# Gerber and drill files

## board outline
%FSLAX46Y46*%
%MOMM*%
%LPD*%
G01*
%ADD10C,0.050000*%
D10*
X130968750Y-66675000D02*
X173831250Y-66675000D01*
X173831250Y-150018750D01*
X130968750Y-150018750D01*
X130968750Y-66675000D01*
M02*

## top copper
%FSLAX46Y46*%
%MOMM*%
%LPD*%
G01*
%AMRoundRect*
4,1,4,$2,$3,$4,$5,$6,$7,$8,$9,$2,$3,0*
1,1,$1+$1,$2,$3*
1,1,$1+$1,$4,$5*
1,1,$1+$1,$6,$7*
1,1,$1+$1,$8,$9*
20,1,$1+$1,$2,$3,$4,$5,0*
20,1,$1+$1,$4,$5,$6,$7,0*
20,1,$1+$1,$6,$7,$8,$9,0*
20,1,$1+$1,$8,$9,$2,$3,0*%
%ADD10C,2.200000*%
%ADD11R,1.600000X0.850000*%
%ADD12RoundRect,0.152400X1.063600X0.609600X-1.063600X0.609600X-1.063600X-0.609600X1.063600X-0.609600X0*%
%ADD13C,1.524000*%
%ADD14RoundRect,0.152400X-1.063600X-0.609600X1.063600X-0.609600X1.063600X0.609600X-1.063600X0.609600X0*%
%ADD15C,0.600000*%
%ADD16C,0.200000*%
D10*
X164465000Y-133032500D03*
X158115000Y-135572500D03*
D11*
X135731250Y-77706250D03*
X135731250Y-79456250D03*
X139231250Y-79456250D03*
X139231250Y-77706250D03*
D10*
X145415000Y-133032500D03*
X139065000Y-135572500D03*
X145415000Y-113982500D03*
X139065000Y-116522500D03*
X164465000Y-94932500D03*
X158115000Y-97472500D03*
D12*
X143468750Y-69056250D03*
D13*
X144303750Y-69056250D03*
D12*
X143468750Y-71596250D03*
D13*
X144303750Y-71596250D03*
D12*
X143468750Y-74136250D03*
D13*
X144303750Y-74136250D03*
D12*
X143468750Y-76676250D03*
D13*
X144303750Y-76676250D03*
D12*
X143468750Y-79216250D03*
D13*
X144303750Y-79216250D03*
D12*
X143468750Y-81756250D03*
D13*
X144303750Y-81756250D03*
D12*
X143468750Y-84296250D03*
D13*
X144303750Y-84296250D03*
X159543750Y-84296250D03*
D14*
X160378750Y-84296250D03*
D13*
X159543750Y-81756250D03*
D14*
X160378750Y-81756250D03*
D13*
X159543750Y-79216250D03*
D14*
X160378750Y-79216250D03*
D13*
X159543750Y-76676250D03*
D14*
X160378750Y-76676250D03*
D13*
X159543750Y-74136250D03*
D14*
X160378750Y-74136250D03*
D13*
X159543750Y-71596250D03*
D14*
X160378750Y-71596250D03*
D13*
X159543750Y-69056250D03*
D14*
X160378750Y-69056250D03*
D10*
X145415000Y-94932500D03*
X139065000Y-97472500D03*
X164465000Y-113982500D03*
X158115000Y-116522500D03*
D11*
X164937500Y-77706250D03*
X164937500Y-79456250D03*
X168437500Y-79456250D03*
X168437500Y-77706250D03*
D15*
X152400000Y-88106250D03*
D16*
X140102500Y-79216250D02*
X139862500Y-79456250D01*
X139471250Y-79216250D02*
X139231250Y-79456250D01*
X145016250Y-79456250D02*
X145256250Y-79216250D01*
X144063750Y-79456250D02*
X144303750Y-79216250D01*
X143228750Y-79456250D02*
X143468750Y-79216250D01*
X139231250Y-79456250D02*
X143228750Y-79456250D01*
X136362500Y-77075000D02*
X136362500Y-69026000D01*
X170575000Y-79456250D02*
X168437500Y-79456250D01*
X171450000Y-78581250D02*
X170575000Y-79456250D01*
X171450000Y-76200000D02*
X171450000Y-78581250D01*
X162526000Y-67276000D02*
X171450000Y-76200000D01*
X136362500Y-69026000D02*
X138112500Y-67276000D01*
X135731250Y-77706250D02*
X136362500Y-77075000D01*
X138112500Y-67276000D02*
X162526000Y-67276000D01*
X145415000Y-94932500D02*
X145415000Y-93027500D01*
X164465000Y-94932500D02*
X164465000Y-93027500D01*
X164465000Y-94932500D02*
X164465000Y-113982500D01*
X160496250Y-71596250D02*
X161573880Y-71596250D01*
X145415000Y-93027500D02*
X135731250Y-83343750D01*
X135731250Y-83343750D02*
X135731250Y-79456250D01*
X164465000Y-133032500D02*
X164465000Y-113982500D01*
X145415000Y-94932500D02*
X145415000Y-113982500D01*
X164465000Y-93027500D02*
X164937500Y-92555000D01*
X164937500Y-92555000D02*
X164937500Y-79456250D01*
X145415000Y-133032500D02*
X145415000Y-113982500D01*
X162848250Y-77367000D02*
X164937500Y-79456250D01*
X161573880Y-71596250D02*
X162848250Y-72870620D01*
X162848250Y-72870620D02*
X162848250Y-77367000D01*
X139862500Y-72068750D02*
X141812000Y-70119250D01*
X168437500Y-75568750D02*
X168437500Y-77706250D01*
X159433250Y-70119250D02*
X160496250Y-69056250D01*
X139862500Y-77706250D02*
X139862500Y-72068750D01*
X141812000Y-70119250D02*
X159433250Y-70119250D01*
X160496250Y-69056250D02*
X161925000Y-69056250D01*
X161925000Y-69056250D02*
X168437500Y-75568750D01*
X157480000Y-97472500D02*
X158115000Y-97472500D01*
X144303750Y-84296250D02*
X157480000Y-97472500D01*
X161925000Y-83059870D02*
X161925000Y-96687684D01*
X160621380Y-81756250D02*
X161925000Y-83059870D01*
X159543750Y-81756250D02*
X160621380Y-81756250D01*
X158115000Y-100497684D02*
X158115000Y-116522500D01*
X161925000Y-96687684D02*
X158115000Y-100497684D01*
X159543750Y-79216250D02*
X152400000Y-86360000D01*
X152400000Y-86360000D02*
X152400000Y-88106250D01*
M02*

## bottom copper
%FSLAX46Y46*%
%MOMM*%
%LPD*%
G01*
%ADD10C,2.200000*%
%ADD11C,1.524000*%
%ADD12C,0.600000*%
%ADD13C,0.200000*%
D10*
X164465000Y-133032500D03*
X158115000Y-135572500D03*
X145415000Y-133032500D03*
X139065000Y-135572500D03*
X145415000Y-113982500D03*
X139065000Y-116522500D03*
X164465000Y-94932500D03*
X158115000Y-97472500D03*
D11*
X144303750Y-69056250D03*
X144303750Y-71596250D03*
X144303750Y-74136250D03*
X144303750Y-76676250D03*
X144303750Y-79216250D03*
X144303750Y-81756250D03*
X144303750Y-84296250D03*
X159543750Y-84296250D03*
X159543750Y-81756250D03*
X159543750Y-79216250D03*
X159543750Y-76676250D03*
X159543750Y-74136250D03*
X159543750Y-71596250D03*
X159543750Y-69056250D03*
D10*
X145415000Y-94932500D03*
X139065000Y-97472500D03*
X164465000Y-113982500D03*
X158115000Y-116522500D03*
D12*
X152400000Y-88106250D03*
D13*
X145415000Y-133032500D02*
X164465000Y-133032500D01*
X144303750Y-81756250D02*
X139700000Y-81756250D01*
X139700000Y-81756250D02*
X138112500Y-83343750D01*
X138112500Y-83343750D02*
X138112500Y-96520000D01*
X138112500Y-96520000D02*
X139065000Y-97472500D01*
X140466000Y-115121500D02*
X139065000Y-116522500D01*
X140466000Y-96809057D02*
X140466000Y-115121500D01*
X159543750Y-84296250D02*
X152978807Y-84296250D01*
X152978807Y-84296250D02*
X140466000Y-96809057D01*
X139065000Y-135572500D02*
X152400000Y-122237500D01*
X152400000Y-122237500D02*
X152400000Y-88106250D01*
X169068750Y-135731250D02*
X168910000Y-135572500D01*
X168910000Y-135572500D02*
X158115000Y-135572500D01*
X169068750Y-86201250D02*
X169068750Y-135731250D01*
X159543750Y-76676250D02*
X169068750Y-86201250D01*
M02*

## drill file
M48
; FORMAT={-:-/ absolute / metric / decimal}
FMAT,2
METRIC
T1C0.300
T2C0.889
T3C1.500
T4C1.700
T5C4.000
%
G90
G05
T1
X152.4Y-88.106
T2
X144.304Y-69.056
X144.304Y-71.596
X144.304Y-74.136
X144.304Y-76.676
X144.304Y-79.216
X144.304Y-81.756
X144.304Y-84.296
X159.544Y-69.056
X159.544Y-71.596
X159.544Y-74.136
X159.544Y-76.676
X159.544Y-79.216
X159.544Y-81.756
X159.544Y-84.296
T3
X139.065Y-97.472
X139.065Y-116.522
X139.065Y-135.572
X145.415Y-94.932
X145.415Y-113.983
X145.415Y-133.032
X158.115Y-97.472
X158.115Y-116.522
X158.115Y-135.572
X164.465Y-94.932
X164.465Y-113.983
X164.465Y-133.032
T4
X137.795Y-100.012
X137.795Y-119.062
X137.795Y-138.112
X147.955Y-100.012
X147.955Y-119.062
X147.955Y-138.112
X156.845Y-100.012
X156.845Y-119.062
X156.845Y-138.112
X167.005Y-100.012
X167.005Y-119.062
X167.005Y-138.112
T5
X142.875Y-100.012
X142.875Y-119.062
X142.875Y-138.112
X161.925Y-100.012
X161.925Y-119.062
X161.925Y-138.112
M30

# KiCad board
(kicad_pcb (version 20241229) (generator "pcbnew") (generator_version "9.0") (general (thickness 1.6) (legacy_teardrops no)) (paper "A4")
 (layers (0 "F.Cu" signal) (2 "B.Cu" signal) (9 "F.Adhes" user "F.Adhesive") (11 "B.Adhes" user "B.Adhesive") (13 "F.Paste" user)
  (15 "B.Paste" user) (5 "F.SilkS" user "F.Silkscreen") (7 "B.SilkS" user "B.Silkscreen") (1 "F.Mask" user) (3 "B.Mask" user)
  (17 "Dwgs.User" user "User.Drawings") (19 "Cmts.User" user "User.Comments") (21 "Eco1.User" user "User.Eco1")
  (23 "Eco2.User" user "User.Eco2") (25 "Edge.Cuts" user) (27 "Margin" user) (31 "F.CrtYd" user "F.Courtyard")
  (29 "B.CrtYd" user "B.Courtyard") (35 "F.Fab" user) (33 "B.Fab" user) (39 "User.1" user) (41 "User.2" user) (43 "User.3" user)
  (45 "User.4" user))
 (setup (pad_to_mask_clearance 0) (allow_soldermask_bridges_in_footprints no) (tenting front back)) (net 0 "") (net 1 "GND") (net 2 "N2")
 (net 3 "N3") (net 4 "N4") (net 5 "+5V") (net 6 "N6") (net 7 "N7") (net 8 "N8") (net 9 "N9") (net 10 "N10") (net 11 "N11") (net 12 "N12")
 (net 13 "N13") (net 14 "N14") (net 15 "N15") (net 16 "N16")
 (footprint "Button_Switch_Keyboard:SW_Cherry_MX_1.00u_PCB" (layer "F.Cu") (at 164.465 133.0325)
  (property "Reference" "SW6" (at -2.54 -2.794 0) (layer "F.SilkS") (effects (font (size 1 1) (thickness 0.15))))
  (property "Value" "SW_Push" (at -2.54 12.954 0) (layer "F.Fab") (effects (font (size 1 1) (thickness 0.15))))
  (pad "" np_thru_hole circle (at -7.62 5.08) (size 1.7 1.7) (drill 1.7) (layers "*.Cu" "*.Mask"))
  (pad "" np_thru_hole circle (at -2.54 5.08) (size 4 4) (drill 4) (layers "*.Cu" "*.Mask"))
  (pad "" np_thru_hole circle (at 2.54 5.08) (size 1.7 1.7) (drill 1.7) (layers "*.Cu" "*.Mask"))
  (pad "1" thru_hole circle (at 0 0) (size 2.2 2.2) (drill 1.5) (layers "*.Cu" "*.Mask") (remove_unused_layers no) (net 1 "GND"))
  (pad "2" thru_hole circle (at -6.35 2.54) (size 2.2 2.2) (drill 1.5) (layers "*.Cu" "*.Mask") (remove_unused_layers no) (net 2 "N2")))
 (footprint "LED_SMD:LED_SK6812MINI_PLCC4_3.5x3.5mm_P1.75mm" (layer "F.Cu") (at 137.48125 78.58125)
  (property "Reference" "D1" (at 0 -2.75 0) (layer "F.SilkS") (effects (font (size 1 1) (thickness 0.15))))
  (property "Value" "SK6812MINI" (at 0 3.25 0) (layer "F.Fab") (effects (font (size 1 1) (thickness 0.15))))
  (pad "1" smd rect (at -1.75 -0.875) (size 1.6 0.85) (layers "F.Cu" "F.Mask" "F.Paste") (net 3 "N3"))
  (pad "2" smd rect (at -1.75 0.875) (size 1.6 0.85) (layers "F.Cu" "F.Mask" "F.Paste") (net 1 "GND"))
  (pad "3" smd rect (at 1.75 0.875) (size 1.6 0.85) (layers "F.Cu" "F.Mask" "F.Paste") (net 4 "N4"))
  (pad "4" smd rect (at 1.75 -0.875) (size 1.6 0.85) (layers "F.Cu" "F.Mask" "F.Paste") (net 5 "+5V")))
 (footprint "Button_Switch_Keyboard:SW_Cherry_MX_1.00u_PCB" (layer "F.Cu") (at 145.415 133.0325)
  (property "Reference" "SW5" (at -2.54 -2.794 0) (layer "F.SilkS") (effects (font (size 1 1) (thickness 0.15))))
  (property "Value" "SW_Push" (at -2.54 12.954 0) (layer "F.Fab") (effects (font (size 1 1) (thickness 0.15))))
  (pad "" np_thru_hole circle (at -7.62 5.08) (size 1.7 1.7) (drill 1.7) (layers "*.Cu" "*.Mask"))
  (pad "" np_thru_hole circle (at -2.54 5.08) (size 4 4) (drill 4) (layers "*.Cu" "*.Mask"))
  (pad "" np_thru_hole circle (at 2.54 5.08) (size 1.7 1.7) (drill 1.7) (layers "*.Cu" "*.Mask"))
  (pad "1" thru_hole circle (at 0 0) (size 2.2 2.2) (drill 1.5) (layers "*.Cu" "*.Mask") (remove_unused_layers no) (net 1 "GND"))
  (pad "2" thru_hole circle (at -6.35 2.54) (size 2.2 2.2) (drill 1.5) (layers "*.Cu" "*.Mask") (remove_unused_layers no) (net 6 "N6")))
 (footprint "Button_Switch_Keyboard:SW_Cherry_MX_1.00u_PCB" (layer "F.Cu") (at 145.415 113.9825)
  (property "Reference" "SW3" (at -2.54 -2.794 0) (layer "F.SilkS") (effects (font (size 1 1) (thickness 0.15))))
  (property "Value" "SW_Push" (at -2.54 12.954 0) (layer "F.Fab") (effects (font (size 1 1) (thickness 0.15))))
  (pad "" np_thru_hole circle (at -7.62 5.08) (size 1.7 1.7) (drill 1.7) (layers "*.Cu" "*.Mask"))
  (pad "" np_thru_hole circle (at -2.54 5.08) (size 4 4) (drill 4) (layers "*.Cu" "*.Mask"))
  (pad "" np_thru_hole circle (at 2.54 5.08) (size 1.7 1.7) (drill 1.7) (layers "*.Cu" "*.Mask"))
  (pad "1" thru_hole circle (at 0 0) (size 2.2 2.2) (drill 1.5) (layers "*.Cu" "*.Mask") (remove_unused_layers no) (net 1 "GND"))
  (pad "2" thru_hole circle (at -6.35 2.54) (size 2.2 2.2) (drill 1.5) (layers "*.Cu" "*.Mask") (remove_unused_layers no) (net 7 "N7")))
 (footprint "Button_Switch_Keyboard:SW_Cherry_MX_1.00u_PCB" (layer "F.Cu") (at 164.465 94.9325)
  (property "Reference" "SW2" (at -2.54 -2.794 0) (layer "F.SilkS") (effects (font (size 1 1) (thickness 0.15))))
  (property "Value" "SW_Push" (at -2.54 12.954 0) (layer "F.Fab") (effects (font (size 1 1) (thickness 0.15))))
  (pad "" np_thru_hole circle (at -7.62 5.08) (size 1.7 1.7) (drill 1.7) (layers "*.Cu" "*.Mask"))
  (pad "" np_thru_hole circle (at -2.54 5.08) (size 4 4) (drill 4) (layers "*.Cu" "*.Mask"))
  (pad "" np_thru_hole circle (at 2.54 5.08) (size 1.7 1.7) (drill 1.7) (layers "*.Cu" "*.Mask"))
  (pad "1" thru_hole circle (at 0 0) (size 2.2 2.2) (drill 1.5) (layers "*.Cu" "*.Mask") (remove_unused_layers no) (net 1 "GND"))
  (pad "2" thru_hole circle (at -6.35 2.54) (size 2.2 2.2) (drill 1.5) (layers "*.Cu" "*.Mask") (remove_unused_layers no) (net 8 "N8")))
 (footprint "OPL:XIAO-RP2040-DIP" (layer "F.Cu") (at 151.92375 76.67625)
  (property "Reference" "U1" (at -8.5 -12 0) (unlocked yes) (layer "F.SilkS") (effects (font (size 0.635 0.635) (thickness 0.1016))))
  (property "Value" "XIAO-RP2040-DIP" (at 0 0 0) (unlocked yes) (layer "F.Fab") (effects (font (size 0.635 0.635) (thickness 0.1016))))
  (pad "1" smd roundrect (at -8.455 -7.62 180) (size 2.432 1.524) (layers "F.Cu" "F.Mask") (roundrect_rratio 0.1) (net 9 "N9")
   (thermal_bridge_angle 45))
  (pad "1" thru_hole circle (at -7.62 -7.62 180) (size 1.524 1.524) (drill 0.889) (layers "*.Cu" "*.Mask") (remove_unused_layers no)
   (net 9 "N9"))
  (pad "2" smd roundrect (at -8.455 -5.08 180) (size 2.432 1.524) (layers "F.Cu" "F.Mask") (roundrect_rratio 0.1) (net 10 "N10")
   (thermal_bridge_angle 45))
  (pad "2" thru_hole circle (at -7.62 -5.08 180) (size 1.524 1.524) (drill 0.889) (layers "*.Cu" "*.Mask") (remove_unused_layers no)
   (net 10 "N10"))
  (pad "3" smd roundrect (at -8.455 -2.54 180) (size 2.432 1.524) (layers "F.Cu" "F.Mask") (roundrect_rratio 0.1) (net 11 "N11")
   (thermal_bridge_angle 45))
  (pad "3" thru_hole circle (at -7.62 -2.54 180) (size 1.524 1.524) (drill 0.889) (layers "*.Cu" "*.Mask") (remove_unused_layers no)
   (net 11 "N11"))
  (pad "4" smd roundrect (at -8.455 0 180) (size 2.432 1.524) (layers "F.Cu" "F.Mask") (roundrect_rratio 0.1) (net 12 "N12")
   (thermal_bridge_angle 45))
  (pad "4" thru_hole circle (at -7.62 0 180) (size 1.524 1.524) (drill 0.889) (layers "*.Cu" "*.Mask") (remove_unused_layers no)
   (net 12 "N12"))
  (pad "5" smd roundrect (at -8.455 2.54 180) (size 2.432 1.524) (layers "F.Cu" "F.Mask") (roundrect_rratio 0.1) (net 4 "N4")
   (thermal_bridge_angle 45))
  (pad "5" thru_hole circle (at -7.62 2.54 180) (size 1.524 1.524) (drill 0.889) (layers "*.Cu" "*.Mask") (remove_unused_layers no)
   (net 4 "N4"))
  (pad "6" smd roundrect (at -8.455 5.08 180) (size 2.432 1.524) (layers "F.Cu" "F.Mask") (roundrect_rratio 0.1) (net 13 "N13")
   (thermal_bridge_angle 45))
  (pad "6" thru_hole circle (at -7.62 5.08 180) (size 1.524 1.524) (drill 0.889) (layers "*.Cu" "*.Mask") (remove_unused_layers no)
   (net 13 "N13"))
  (pad "7" smd roundrect (at -8.455 7.62 180) (size 2.432 1.524) (layers "F.Cu" "F.Mask") (roundrect_rratio 0.1) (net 8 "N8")
   (thermal_bridge_angle 45))
  (pad "7" thru_hole circle (at -7.62 7.62 180) (size 1.524 1.524) (drill 0.889) (layers "*.Cu" "*.Mask") (remove_unused_layers no)
   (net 8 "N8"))
  (pad "8" thru_hole circle (at 7.62 7.62) (size 1.524 1.524) (drill 0.889) (layers "*.Cu" "*.Mask") (remove_unused_layers no) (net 7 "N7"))
  (pad "8" smd roundrect (at 8.455 7.62) (size 2.432 1.524) (layers "F.Cu" "F.Mask") (roundrect_rratio 0.1) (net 7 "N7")
   (thermal_bridge_angle 45))
  (pad "9" thru_hole circle (at 7.62 5.08) (size 1.524 1.524) (drill 0.889) (layers "*.Cu" "*.Mask") (remove_unused_layers no)
   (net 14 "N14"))
  (pad "9" smd roundrect (at 8.455 5.08) (size 2.432 1.524) (layers "F.Cu" "F.Mask") (roundrect_rratio 0.1) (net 14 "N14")
   (thermal_bridge_angle 45))
  (pad "10" thru_hole circle (at 7.62 2.54) (size 1.524 1.524) (drill 0.889) (layers "*.Cu" "*.Mask") (remove_unused_layers no) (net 6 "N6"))
  (pad "10" smd roundrect (at 8.455 2.54) (size 2.432 1.524) (layers "F.Cu" "F.Mask") (roundrect_rratio 0.1) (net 6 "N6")
   (thermal_bridge_angle 45))
  (pad "11" thru_hole circle (at 7.62 0) (size 1.524 1.524) (drill 0.889) (layers "*.Cu" "*.Mask") (remove_unused_layers no) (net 2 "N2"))
  (pad "11" smd roundrect (at 8.455 0) (size 2.432 1.524) (layers "F.Cu" "F.Mask") (roundrect_rratio 0.1) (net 2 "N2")
   (thermal_bridge_angle 45))
  (pad "12" thru_hole circle (at 7.62 -2.54) (size 1.524 1.524) (drill 0.889) (layers "*.Cu" "*.Mask") (remove_unused_layers no)
   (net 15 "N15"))
  (pad "12" smd roundrect (at 8.455 -2.54) (size 2.432 1.524) (layers "F.Cu" "F.Mask") (roundrect_rratio 0.1) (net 15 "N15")
   (thermal_bridge_angle 45))
  (pad "13" thru_hole circle (at 7.62 -5.08) (size 1.524 1.524) (drill 0.889) (layers "*.Cu" "*.Mask") (remove_unused_layers no)
   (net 1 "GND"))
  (pad "13" smd roundrect (at 8.455 -5.08) (size 2.432 1.524) (layers "F.Cu" "F.Mask") (roundrect_rratio 0.1) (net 1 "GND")
   (thermal_bridge_angle 45))
  (pad "14" thru_hole circle (at 7.62 -7.62) (size 1.524 1.524) (drill 0.889) (layers "*.Cu" "*.Mask") (remove_unused_layers no)
   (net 5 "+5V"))
  (pad "14" smd roundrect (at 8.455 -7.62) (size 2.432 1.524) (layers "F.Cu" "F.Mask") (roundrect_rratio 0.1) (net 5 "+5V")
   (thermal_bridge_angle 45)))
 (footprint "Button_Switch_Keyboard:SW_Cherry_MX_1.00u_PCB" (layer "F.Cu") (at 145.415 94.9325)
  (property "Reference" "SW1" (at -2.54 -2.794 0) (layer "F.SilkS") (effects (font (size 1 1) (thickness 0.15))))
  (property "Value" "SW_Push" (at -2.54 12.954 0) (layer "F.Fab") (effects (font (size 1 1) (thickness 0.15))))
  (pad "" np_thru_hole circle (at -7.62 5.08) (size 1.7 1.7) (drill 1.7) (layers "*.Cu" "*.Mask"))
  (pad "" np_thru_hole circle (at -2.54 5.08) (size 4 4) (drill 4) (layers "*.Cu" "*.Mask"))
  (pad "" np_thru_hole circle (at 2.54 5.08) (size 1.7 1.7) (drill 1.7) (layers "*.Cu" "*.Mask"))
  (pad "1" thru_hole circle (at 0 0) (size 2.2 2.2) (drill 1.5) (layers "*.Cu" "*.Mask") (remove_unused_layers no) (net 1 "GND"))
  (pad "2" thru_hole circle (at -6.35 2.54) (size 2.2 2.2) (drill 1.5) (layers "*.Cu" "*.Mask") (remove_unused_layers no) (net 13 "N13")))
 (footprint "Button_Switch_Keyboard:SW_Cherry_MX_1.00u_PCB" (layer "F.Cu") (at 164.465 113.9825)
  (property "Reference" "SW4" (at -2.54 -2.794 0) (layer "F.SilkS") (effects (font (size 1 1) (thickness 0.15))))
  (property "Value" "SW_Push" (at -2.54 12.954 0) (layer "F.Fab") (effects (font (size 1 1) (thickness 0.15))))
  (pad "" np_thru_hole circle (at -7.62 5.08) (size 1.7 1.7) (drill 1.7) (layers "*.Cu" "*.Mask"))
  (pad "" np_thru_hole circle (at -2.54 5.08) (size 4 4) (drill 4) (layers "*.Cu" "*.Mask"))
  (pad "" np_thru_hole circle (at 2.54 5.08) (size 1.7 1.7) (drill 1.7) (layers "*.Cu" "*.Mask"))
  (pad "1" thru_hole circle (at 0 0) (size 2.2 2.2) (drill 1.5) (layers "*.Cu" "*.Mask") (remove_unused_layers no) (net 1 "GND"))
  (pad "2" thru_hole circle (at -6.35 2.54) (size 2.2 2.2) (drill 1.5) (layers "*.Cu" "*.Mask") (remove_unused_layers no) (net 14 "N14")))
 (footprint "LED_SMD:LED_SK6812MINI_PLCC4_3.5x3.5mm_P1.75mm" (layer "F.Cu") (at 166.6875 78.58125)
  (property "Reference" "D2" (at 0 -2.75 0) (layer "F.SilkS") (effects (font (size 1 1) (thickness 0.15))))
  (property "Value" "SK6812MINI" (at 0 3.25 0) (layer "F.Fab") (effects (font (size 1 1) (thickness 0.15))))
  (pad "1" smd rect (at -1.75 -0.875) (size 1.6 0.85) (layers "F.Cu" "F.Mask" "F.Paste") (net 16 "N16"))
  (pad "2" smd rect (at -1.75 0.875) (size 1.6 0.85) (layers "F.Cu" "F.Mask" "F.Paste") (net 1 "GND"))
  (pad "3" smd rect (at 1.75 0.875) (size 1.6 0.85) (layers "F.Cu" "F.Mask" "F.Paste") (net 3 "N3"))
  (pad "4" smd rect (at 1.75 -0.875) (size 1.6 0.85) (layers "F.Cu" "F.Mask" "F.Paste") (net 5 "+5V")))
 (gr_rect (start 130.96875 66.675) (end 173.83125 150.01875) (stroke (width 0.05) (type default)) (fill no) (layer "Edge.Cuts"))
 (segment (start 140.1025 79.21625) (end 139.8625 79.45625) (width 0.2) (layer "F.Cu") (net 4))
 (segment (start 139.47125 79.21625) (end 139.23125 79.45625) (width 0.2) (layer "F.Cu") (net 4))
 (segment (start 145.01625 79.45625) (end 145.25625 79.21625) (width 0.2) (layer "F.Cu") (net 4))
 (segment (start 144.06375 79.45625) (end 144.30375 79.21625) (width 0.2) (layer "F.Cu") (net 4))
 (segment (start 143.22875 79.45625) (end 143.46875 79.21625) (width 0.2) (layer "F.Cu") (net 4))
 (segment (start 139.23125 79.45625) (end 143.22875 79.45625) (width 0.2) (layer "F.Cu") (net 4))
 (segment (start 136.3625 77.075) (end 136.3625 69.026) (width 0.2) (layer "F.Cu") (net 3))
 (segment (start 170.575 79.45625) (end 168.4375 79.45625) (width 0.2) (layer "F.Cu") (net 3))
 (segment (start 171.45 78.58125) (end 170.575 79.45625) (width 0.2) (layer "F.Cu") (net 3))
 (segment (start 171.45 76.2) (end 171.45 78.58125) (width 0.2) (layer "F.Cu") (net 3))
 (segment (start 162.526 67.276) (end 171.45 76.2) (width 0.2) (layer "F.Cu") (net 3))
 (segment (start 136.3625 69.026) (end 138.1125 67.276) (width 0.2) (layer "F.Cu") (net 3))
 (segment (start 135.73125 77.70625) (end 136.3625 77.075) (width 0.2) (layer "F.Cu") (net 3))
 (segment (start 138.1125 67.276) (end 162.526 67.276) (width 0.2) (layer "F.Cu") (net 3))
 (segment (start 145.415 94.9325) (end 145.415 93.0275) (width 0.2) (layer "F.Cu") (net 1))
 (segment (start 164.465 94.9325) (end 164.465 93.0275) (width 0.2) (layer "F.Cu") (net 1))
 (segment (start 164.465 94.9325) (end 164.465 113.9825) (width 0.2) (layer "F.Cu") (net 1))
 (segment (start 160.49625 71.59625) (end 161.57388 71.59625) (width 0.2) (layer "F.Cu") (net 1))
 (segment (start 145.415 93.0275) (end 135.73125 83.34375) (width 0.2) (layer "F.Cu") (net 1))
 (segment (start 135.73125 83.34375) (end 135.73125 79.45625) (width 0.2) (layer "F.Cu") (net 1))
 (segment (start 164.465 133.0325) (end 164.465 113.9825) (width 0.2) (layer "F.Cu") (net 1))
 (segment (start 145.415 94.9325) (end 145.415 113.9825) (width 0.2) (layer "F.Cu") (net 1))
 (segment (start 164.465 93.0275) (end 164.9375 92.555) (width 0.2) (layer "F.Cu") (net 1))
 (segment (start 164.9375 92.555) (end 164.9375 79.45625) (width 0.2) (layer "F.Cu") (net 1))
 (segment (start 145.415 133.0325) (end 145.415 113.9825) (width 0.2) (layer "F.Cu") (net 1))
 (segment (start 162.84825 77.367) (end 164.9375 79.45625) (width 0.2) (layer "F.Cu") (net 1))
 (segment (start 161.57388 71.59625) (end 162.84825 72.87062) (width 0.2) (layer "F.Cu") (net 1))
 (segment (start 162.84825 72.87062) (end 162.84825 77.367) (width 0.2) (layer "F.Cu") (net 1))
 (segment (start 145.415 133.0325) (end 164.465 133.0325) (width 0.2) (layer "B.Cu") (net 1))
 (segment (start 139.8625 72.06875) (end 141.812 70.11925) (width 0.2) (layer "F.Cu") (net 5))
 (segment (start 168.4375 75.56875) (end 168.4375 77.70625) (width 0.2) (layer "F.Cu") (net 5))
 (segment (start 159.43325 70.11925) (end 160.49625 69.05625) (width 0.2) (layer "F.Cu") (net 5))
 (segment (start 139.8625 77.70625) (end 139.8625 72.06875) (width 0.2) (layer "F.Cu") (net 5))
 (segment (start 141.812 70.11925) (end 159.43325 70.11925) (width 0.2) (layer "F.Cu") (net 5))
 (segment (start 160.49625 69.05625) (end 161.925 69.05625) (width 0.2) (layer "F.Cu") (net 5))
 (segment (start 161.925 69.05625) (end 168.4375 75.56875) (width 0.2) (layer "F.Cu") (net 5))
 (segment (start 144.30375 81.75625) (end 139.7 81.75625) (width 0.2) (layer "B.Cu") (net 13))
 (segment (start 139.7 81.75625) (end 138.1125 83.34375) (width 0.2) (layer "B.Cu") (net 13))
 (segment (start 138.1125 83.34375) (end 138.1125 96.52) (width 0.2) (layer "B.Cu") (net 13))
 (segment (start 138.1125 96.52) (end 139.065 97.4725) (width 0.2) (layer "B.Cu") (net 13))
 (segment (start 157.48 97.4725) (end 158.115 97.4725) (width 0.2) (layer "F.Cu") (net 8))
 (segment (start 144.30375 84.29625) (end 157.48 97.4725) (width 0.2) (layer "F.Cu") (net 8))
 (segment (start 140.466 115.1215) (end 139.065 116.5225) (width 0.2) (layer "B.Cu") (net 7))
 (segment (start 140.466 96.809057) (end 140.466 115.1215) (width 0.2) (layer "B.Cu") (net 7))
 (segment (start 159.54375 84.29625) (end 152.978807 84.29625) (width 0.2) (layer "B.Cu") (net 7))
 (segment (start 152.978807 84.29625) (end 140.466 96.809057) (width 0.2) (layer "B.Cu") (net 7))
 (segment (start 161.925 83.05987) (end 161.925 96.687684) (width 0.2) (layer "F.Cu") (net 14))
 (segment (start 160.62138 81.75625) (end 161.925 83.05987) (width 0.2) (layer "F.Cu") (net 14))
 (segment (start 159.54375 81.75625) (end 160.62138 81.75625) (width 0.2) (layer "F.Cu") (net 14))
 (segment (start 158.115 100.497684) (end 158.115 116.5225) (width 0.2) (layer "F.Cu") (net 14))
 (segment (start 161.925 96.687684) (end 158.115 100.497684) (width 0.2) (layer "F.Cu") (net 14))
 (segment (start 159.54375 79.21625) (end 152.4 86.36) (width 0.2) (layer "F.Cu") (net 6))
 (segment (start 152.4 86.36) (end 152.4 88.10625) (width 0.2) (layer "F.Cu") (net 6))
 (via (at 152.4 88.10625) (size 0.6) (drill 0.3) (layers "F.Cu" "B.Cu") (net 6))
 (segment (start 139.065 135.5725) (end 152.4 122.2375) (width 0.2) (layer "B.Cu") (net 6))
 (segment (start 152.4 122.2375) (end 152.4 88.10625) (width 0.2) (layer "B.Cu") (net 6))
 (segment (start 169.06875 135.73125) (end 168.91 135.5725) (width 0.2) (layer "B.Cu") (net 2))
 (segment (start 168.91 135.5725) (end 158.115 135.5725) (width 0.2) (layer "B.Cu") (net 2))
 (segment (start 169.06875 86.20125) (end 169.06875 135.73125) (width 0.2) (layer "B.Cu") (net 2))
 (segment (start 159.54375 76.67625) (end 169.06875 86.20125) (width 0.2) (layer "B.Cu") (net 2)))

